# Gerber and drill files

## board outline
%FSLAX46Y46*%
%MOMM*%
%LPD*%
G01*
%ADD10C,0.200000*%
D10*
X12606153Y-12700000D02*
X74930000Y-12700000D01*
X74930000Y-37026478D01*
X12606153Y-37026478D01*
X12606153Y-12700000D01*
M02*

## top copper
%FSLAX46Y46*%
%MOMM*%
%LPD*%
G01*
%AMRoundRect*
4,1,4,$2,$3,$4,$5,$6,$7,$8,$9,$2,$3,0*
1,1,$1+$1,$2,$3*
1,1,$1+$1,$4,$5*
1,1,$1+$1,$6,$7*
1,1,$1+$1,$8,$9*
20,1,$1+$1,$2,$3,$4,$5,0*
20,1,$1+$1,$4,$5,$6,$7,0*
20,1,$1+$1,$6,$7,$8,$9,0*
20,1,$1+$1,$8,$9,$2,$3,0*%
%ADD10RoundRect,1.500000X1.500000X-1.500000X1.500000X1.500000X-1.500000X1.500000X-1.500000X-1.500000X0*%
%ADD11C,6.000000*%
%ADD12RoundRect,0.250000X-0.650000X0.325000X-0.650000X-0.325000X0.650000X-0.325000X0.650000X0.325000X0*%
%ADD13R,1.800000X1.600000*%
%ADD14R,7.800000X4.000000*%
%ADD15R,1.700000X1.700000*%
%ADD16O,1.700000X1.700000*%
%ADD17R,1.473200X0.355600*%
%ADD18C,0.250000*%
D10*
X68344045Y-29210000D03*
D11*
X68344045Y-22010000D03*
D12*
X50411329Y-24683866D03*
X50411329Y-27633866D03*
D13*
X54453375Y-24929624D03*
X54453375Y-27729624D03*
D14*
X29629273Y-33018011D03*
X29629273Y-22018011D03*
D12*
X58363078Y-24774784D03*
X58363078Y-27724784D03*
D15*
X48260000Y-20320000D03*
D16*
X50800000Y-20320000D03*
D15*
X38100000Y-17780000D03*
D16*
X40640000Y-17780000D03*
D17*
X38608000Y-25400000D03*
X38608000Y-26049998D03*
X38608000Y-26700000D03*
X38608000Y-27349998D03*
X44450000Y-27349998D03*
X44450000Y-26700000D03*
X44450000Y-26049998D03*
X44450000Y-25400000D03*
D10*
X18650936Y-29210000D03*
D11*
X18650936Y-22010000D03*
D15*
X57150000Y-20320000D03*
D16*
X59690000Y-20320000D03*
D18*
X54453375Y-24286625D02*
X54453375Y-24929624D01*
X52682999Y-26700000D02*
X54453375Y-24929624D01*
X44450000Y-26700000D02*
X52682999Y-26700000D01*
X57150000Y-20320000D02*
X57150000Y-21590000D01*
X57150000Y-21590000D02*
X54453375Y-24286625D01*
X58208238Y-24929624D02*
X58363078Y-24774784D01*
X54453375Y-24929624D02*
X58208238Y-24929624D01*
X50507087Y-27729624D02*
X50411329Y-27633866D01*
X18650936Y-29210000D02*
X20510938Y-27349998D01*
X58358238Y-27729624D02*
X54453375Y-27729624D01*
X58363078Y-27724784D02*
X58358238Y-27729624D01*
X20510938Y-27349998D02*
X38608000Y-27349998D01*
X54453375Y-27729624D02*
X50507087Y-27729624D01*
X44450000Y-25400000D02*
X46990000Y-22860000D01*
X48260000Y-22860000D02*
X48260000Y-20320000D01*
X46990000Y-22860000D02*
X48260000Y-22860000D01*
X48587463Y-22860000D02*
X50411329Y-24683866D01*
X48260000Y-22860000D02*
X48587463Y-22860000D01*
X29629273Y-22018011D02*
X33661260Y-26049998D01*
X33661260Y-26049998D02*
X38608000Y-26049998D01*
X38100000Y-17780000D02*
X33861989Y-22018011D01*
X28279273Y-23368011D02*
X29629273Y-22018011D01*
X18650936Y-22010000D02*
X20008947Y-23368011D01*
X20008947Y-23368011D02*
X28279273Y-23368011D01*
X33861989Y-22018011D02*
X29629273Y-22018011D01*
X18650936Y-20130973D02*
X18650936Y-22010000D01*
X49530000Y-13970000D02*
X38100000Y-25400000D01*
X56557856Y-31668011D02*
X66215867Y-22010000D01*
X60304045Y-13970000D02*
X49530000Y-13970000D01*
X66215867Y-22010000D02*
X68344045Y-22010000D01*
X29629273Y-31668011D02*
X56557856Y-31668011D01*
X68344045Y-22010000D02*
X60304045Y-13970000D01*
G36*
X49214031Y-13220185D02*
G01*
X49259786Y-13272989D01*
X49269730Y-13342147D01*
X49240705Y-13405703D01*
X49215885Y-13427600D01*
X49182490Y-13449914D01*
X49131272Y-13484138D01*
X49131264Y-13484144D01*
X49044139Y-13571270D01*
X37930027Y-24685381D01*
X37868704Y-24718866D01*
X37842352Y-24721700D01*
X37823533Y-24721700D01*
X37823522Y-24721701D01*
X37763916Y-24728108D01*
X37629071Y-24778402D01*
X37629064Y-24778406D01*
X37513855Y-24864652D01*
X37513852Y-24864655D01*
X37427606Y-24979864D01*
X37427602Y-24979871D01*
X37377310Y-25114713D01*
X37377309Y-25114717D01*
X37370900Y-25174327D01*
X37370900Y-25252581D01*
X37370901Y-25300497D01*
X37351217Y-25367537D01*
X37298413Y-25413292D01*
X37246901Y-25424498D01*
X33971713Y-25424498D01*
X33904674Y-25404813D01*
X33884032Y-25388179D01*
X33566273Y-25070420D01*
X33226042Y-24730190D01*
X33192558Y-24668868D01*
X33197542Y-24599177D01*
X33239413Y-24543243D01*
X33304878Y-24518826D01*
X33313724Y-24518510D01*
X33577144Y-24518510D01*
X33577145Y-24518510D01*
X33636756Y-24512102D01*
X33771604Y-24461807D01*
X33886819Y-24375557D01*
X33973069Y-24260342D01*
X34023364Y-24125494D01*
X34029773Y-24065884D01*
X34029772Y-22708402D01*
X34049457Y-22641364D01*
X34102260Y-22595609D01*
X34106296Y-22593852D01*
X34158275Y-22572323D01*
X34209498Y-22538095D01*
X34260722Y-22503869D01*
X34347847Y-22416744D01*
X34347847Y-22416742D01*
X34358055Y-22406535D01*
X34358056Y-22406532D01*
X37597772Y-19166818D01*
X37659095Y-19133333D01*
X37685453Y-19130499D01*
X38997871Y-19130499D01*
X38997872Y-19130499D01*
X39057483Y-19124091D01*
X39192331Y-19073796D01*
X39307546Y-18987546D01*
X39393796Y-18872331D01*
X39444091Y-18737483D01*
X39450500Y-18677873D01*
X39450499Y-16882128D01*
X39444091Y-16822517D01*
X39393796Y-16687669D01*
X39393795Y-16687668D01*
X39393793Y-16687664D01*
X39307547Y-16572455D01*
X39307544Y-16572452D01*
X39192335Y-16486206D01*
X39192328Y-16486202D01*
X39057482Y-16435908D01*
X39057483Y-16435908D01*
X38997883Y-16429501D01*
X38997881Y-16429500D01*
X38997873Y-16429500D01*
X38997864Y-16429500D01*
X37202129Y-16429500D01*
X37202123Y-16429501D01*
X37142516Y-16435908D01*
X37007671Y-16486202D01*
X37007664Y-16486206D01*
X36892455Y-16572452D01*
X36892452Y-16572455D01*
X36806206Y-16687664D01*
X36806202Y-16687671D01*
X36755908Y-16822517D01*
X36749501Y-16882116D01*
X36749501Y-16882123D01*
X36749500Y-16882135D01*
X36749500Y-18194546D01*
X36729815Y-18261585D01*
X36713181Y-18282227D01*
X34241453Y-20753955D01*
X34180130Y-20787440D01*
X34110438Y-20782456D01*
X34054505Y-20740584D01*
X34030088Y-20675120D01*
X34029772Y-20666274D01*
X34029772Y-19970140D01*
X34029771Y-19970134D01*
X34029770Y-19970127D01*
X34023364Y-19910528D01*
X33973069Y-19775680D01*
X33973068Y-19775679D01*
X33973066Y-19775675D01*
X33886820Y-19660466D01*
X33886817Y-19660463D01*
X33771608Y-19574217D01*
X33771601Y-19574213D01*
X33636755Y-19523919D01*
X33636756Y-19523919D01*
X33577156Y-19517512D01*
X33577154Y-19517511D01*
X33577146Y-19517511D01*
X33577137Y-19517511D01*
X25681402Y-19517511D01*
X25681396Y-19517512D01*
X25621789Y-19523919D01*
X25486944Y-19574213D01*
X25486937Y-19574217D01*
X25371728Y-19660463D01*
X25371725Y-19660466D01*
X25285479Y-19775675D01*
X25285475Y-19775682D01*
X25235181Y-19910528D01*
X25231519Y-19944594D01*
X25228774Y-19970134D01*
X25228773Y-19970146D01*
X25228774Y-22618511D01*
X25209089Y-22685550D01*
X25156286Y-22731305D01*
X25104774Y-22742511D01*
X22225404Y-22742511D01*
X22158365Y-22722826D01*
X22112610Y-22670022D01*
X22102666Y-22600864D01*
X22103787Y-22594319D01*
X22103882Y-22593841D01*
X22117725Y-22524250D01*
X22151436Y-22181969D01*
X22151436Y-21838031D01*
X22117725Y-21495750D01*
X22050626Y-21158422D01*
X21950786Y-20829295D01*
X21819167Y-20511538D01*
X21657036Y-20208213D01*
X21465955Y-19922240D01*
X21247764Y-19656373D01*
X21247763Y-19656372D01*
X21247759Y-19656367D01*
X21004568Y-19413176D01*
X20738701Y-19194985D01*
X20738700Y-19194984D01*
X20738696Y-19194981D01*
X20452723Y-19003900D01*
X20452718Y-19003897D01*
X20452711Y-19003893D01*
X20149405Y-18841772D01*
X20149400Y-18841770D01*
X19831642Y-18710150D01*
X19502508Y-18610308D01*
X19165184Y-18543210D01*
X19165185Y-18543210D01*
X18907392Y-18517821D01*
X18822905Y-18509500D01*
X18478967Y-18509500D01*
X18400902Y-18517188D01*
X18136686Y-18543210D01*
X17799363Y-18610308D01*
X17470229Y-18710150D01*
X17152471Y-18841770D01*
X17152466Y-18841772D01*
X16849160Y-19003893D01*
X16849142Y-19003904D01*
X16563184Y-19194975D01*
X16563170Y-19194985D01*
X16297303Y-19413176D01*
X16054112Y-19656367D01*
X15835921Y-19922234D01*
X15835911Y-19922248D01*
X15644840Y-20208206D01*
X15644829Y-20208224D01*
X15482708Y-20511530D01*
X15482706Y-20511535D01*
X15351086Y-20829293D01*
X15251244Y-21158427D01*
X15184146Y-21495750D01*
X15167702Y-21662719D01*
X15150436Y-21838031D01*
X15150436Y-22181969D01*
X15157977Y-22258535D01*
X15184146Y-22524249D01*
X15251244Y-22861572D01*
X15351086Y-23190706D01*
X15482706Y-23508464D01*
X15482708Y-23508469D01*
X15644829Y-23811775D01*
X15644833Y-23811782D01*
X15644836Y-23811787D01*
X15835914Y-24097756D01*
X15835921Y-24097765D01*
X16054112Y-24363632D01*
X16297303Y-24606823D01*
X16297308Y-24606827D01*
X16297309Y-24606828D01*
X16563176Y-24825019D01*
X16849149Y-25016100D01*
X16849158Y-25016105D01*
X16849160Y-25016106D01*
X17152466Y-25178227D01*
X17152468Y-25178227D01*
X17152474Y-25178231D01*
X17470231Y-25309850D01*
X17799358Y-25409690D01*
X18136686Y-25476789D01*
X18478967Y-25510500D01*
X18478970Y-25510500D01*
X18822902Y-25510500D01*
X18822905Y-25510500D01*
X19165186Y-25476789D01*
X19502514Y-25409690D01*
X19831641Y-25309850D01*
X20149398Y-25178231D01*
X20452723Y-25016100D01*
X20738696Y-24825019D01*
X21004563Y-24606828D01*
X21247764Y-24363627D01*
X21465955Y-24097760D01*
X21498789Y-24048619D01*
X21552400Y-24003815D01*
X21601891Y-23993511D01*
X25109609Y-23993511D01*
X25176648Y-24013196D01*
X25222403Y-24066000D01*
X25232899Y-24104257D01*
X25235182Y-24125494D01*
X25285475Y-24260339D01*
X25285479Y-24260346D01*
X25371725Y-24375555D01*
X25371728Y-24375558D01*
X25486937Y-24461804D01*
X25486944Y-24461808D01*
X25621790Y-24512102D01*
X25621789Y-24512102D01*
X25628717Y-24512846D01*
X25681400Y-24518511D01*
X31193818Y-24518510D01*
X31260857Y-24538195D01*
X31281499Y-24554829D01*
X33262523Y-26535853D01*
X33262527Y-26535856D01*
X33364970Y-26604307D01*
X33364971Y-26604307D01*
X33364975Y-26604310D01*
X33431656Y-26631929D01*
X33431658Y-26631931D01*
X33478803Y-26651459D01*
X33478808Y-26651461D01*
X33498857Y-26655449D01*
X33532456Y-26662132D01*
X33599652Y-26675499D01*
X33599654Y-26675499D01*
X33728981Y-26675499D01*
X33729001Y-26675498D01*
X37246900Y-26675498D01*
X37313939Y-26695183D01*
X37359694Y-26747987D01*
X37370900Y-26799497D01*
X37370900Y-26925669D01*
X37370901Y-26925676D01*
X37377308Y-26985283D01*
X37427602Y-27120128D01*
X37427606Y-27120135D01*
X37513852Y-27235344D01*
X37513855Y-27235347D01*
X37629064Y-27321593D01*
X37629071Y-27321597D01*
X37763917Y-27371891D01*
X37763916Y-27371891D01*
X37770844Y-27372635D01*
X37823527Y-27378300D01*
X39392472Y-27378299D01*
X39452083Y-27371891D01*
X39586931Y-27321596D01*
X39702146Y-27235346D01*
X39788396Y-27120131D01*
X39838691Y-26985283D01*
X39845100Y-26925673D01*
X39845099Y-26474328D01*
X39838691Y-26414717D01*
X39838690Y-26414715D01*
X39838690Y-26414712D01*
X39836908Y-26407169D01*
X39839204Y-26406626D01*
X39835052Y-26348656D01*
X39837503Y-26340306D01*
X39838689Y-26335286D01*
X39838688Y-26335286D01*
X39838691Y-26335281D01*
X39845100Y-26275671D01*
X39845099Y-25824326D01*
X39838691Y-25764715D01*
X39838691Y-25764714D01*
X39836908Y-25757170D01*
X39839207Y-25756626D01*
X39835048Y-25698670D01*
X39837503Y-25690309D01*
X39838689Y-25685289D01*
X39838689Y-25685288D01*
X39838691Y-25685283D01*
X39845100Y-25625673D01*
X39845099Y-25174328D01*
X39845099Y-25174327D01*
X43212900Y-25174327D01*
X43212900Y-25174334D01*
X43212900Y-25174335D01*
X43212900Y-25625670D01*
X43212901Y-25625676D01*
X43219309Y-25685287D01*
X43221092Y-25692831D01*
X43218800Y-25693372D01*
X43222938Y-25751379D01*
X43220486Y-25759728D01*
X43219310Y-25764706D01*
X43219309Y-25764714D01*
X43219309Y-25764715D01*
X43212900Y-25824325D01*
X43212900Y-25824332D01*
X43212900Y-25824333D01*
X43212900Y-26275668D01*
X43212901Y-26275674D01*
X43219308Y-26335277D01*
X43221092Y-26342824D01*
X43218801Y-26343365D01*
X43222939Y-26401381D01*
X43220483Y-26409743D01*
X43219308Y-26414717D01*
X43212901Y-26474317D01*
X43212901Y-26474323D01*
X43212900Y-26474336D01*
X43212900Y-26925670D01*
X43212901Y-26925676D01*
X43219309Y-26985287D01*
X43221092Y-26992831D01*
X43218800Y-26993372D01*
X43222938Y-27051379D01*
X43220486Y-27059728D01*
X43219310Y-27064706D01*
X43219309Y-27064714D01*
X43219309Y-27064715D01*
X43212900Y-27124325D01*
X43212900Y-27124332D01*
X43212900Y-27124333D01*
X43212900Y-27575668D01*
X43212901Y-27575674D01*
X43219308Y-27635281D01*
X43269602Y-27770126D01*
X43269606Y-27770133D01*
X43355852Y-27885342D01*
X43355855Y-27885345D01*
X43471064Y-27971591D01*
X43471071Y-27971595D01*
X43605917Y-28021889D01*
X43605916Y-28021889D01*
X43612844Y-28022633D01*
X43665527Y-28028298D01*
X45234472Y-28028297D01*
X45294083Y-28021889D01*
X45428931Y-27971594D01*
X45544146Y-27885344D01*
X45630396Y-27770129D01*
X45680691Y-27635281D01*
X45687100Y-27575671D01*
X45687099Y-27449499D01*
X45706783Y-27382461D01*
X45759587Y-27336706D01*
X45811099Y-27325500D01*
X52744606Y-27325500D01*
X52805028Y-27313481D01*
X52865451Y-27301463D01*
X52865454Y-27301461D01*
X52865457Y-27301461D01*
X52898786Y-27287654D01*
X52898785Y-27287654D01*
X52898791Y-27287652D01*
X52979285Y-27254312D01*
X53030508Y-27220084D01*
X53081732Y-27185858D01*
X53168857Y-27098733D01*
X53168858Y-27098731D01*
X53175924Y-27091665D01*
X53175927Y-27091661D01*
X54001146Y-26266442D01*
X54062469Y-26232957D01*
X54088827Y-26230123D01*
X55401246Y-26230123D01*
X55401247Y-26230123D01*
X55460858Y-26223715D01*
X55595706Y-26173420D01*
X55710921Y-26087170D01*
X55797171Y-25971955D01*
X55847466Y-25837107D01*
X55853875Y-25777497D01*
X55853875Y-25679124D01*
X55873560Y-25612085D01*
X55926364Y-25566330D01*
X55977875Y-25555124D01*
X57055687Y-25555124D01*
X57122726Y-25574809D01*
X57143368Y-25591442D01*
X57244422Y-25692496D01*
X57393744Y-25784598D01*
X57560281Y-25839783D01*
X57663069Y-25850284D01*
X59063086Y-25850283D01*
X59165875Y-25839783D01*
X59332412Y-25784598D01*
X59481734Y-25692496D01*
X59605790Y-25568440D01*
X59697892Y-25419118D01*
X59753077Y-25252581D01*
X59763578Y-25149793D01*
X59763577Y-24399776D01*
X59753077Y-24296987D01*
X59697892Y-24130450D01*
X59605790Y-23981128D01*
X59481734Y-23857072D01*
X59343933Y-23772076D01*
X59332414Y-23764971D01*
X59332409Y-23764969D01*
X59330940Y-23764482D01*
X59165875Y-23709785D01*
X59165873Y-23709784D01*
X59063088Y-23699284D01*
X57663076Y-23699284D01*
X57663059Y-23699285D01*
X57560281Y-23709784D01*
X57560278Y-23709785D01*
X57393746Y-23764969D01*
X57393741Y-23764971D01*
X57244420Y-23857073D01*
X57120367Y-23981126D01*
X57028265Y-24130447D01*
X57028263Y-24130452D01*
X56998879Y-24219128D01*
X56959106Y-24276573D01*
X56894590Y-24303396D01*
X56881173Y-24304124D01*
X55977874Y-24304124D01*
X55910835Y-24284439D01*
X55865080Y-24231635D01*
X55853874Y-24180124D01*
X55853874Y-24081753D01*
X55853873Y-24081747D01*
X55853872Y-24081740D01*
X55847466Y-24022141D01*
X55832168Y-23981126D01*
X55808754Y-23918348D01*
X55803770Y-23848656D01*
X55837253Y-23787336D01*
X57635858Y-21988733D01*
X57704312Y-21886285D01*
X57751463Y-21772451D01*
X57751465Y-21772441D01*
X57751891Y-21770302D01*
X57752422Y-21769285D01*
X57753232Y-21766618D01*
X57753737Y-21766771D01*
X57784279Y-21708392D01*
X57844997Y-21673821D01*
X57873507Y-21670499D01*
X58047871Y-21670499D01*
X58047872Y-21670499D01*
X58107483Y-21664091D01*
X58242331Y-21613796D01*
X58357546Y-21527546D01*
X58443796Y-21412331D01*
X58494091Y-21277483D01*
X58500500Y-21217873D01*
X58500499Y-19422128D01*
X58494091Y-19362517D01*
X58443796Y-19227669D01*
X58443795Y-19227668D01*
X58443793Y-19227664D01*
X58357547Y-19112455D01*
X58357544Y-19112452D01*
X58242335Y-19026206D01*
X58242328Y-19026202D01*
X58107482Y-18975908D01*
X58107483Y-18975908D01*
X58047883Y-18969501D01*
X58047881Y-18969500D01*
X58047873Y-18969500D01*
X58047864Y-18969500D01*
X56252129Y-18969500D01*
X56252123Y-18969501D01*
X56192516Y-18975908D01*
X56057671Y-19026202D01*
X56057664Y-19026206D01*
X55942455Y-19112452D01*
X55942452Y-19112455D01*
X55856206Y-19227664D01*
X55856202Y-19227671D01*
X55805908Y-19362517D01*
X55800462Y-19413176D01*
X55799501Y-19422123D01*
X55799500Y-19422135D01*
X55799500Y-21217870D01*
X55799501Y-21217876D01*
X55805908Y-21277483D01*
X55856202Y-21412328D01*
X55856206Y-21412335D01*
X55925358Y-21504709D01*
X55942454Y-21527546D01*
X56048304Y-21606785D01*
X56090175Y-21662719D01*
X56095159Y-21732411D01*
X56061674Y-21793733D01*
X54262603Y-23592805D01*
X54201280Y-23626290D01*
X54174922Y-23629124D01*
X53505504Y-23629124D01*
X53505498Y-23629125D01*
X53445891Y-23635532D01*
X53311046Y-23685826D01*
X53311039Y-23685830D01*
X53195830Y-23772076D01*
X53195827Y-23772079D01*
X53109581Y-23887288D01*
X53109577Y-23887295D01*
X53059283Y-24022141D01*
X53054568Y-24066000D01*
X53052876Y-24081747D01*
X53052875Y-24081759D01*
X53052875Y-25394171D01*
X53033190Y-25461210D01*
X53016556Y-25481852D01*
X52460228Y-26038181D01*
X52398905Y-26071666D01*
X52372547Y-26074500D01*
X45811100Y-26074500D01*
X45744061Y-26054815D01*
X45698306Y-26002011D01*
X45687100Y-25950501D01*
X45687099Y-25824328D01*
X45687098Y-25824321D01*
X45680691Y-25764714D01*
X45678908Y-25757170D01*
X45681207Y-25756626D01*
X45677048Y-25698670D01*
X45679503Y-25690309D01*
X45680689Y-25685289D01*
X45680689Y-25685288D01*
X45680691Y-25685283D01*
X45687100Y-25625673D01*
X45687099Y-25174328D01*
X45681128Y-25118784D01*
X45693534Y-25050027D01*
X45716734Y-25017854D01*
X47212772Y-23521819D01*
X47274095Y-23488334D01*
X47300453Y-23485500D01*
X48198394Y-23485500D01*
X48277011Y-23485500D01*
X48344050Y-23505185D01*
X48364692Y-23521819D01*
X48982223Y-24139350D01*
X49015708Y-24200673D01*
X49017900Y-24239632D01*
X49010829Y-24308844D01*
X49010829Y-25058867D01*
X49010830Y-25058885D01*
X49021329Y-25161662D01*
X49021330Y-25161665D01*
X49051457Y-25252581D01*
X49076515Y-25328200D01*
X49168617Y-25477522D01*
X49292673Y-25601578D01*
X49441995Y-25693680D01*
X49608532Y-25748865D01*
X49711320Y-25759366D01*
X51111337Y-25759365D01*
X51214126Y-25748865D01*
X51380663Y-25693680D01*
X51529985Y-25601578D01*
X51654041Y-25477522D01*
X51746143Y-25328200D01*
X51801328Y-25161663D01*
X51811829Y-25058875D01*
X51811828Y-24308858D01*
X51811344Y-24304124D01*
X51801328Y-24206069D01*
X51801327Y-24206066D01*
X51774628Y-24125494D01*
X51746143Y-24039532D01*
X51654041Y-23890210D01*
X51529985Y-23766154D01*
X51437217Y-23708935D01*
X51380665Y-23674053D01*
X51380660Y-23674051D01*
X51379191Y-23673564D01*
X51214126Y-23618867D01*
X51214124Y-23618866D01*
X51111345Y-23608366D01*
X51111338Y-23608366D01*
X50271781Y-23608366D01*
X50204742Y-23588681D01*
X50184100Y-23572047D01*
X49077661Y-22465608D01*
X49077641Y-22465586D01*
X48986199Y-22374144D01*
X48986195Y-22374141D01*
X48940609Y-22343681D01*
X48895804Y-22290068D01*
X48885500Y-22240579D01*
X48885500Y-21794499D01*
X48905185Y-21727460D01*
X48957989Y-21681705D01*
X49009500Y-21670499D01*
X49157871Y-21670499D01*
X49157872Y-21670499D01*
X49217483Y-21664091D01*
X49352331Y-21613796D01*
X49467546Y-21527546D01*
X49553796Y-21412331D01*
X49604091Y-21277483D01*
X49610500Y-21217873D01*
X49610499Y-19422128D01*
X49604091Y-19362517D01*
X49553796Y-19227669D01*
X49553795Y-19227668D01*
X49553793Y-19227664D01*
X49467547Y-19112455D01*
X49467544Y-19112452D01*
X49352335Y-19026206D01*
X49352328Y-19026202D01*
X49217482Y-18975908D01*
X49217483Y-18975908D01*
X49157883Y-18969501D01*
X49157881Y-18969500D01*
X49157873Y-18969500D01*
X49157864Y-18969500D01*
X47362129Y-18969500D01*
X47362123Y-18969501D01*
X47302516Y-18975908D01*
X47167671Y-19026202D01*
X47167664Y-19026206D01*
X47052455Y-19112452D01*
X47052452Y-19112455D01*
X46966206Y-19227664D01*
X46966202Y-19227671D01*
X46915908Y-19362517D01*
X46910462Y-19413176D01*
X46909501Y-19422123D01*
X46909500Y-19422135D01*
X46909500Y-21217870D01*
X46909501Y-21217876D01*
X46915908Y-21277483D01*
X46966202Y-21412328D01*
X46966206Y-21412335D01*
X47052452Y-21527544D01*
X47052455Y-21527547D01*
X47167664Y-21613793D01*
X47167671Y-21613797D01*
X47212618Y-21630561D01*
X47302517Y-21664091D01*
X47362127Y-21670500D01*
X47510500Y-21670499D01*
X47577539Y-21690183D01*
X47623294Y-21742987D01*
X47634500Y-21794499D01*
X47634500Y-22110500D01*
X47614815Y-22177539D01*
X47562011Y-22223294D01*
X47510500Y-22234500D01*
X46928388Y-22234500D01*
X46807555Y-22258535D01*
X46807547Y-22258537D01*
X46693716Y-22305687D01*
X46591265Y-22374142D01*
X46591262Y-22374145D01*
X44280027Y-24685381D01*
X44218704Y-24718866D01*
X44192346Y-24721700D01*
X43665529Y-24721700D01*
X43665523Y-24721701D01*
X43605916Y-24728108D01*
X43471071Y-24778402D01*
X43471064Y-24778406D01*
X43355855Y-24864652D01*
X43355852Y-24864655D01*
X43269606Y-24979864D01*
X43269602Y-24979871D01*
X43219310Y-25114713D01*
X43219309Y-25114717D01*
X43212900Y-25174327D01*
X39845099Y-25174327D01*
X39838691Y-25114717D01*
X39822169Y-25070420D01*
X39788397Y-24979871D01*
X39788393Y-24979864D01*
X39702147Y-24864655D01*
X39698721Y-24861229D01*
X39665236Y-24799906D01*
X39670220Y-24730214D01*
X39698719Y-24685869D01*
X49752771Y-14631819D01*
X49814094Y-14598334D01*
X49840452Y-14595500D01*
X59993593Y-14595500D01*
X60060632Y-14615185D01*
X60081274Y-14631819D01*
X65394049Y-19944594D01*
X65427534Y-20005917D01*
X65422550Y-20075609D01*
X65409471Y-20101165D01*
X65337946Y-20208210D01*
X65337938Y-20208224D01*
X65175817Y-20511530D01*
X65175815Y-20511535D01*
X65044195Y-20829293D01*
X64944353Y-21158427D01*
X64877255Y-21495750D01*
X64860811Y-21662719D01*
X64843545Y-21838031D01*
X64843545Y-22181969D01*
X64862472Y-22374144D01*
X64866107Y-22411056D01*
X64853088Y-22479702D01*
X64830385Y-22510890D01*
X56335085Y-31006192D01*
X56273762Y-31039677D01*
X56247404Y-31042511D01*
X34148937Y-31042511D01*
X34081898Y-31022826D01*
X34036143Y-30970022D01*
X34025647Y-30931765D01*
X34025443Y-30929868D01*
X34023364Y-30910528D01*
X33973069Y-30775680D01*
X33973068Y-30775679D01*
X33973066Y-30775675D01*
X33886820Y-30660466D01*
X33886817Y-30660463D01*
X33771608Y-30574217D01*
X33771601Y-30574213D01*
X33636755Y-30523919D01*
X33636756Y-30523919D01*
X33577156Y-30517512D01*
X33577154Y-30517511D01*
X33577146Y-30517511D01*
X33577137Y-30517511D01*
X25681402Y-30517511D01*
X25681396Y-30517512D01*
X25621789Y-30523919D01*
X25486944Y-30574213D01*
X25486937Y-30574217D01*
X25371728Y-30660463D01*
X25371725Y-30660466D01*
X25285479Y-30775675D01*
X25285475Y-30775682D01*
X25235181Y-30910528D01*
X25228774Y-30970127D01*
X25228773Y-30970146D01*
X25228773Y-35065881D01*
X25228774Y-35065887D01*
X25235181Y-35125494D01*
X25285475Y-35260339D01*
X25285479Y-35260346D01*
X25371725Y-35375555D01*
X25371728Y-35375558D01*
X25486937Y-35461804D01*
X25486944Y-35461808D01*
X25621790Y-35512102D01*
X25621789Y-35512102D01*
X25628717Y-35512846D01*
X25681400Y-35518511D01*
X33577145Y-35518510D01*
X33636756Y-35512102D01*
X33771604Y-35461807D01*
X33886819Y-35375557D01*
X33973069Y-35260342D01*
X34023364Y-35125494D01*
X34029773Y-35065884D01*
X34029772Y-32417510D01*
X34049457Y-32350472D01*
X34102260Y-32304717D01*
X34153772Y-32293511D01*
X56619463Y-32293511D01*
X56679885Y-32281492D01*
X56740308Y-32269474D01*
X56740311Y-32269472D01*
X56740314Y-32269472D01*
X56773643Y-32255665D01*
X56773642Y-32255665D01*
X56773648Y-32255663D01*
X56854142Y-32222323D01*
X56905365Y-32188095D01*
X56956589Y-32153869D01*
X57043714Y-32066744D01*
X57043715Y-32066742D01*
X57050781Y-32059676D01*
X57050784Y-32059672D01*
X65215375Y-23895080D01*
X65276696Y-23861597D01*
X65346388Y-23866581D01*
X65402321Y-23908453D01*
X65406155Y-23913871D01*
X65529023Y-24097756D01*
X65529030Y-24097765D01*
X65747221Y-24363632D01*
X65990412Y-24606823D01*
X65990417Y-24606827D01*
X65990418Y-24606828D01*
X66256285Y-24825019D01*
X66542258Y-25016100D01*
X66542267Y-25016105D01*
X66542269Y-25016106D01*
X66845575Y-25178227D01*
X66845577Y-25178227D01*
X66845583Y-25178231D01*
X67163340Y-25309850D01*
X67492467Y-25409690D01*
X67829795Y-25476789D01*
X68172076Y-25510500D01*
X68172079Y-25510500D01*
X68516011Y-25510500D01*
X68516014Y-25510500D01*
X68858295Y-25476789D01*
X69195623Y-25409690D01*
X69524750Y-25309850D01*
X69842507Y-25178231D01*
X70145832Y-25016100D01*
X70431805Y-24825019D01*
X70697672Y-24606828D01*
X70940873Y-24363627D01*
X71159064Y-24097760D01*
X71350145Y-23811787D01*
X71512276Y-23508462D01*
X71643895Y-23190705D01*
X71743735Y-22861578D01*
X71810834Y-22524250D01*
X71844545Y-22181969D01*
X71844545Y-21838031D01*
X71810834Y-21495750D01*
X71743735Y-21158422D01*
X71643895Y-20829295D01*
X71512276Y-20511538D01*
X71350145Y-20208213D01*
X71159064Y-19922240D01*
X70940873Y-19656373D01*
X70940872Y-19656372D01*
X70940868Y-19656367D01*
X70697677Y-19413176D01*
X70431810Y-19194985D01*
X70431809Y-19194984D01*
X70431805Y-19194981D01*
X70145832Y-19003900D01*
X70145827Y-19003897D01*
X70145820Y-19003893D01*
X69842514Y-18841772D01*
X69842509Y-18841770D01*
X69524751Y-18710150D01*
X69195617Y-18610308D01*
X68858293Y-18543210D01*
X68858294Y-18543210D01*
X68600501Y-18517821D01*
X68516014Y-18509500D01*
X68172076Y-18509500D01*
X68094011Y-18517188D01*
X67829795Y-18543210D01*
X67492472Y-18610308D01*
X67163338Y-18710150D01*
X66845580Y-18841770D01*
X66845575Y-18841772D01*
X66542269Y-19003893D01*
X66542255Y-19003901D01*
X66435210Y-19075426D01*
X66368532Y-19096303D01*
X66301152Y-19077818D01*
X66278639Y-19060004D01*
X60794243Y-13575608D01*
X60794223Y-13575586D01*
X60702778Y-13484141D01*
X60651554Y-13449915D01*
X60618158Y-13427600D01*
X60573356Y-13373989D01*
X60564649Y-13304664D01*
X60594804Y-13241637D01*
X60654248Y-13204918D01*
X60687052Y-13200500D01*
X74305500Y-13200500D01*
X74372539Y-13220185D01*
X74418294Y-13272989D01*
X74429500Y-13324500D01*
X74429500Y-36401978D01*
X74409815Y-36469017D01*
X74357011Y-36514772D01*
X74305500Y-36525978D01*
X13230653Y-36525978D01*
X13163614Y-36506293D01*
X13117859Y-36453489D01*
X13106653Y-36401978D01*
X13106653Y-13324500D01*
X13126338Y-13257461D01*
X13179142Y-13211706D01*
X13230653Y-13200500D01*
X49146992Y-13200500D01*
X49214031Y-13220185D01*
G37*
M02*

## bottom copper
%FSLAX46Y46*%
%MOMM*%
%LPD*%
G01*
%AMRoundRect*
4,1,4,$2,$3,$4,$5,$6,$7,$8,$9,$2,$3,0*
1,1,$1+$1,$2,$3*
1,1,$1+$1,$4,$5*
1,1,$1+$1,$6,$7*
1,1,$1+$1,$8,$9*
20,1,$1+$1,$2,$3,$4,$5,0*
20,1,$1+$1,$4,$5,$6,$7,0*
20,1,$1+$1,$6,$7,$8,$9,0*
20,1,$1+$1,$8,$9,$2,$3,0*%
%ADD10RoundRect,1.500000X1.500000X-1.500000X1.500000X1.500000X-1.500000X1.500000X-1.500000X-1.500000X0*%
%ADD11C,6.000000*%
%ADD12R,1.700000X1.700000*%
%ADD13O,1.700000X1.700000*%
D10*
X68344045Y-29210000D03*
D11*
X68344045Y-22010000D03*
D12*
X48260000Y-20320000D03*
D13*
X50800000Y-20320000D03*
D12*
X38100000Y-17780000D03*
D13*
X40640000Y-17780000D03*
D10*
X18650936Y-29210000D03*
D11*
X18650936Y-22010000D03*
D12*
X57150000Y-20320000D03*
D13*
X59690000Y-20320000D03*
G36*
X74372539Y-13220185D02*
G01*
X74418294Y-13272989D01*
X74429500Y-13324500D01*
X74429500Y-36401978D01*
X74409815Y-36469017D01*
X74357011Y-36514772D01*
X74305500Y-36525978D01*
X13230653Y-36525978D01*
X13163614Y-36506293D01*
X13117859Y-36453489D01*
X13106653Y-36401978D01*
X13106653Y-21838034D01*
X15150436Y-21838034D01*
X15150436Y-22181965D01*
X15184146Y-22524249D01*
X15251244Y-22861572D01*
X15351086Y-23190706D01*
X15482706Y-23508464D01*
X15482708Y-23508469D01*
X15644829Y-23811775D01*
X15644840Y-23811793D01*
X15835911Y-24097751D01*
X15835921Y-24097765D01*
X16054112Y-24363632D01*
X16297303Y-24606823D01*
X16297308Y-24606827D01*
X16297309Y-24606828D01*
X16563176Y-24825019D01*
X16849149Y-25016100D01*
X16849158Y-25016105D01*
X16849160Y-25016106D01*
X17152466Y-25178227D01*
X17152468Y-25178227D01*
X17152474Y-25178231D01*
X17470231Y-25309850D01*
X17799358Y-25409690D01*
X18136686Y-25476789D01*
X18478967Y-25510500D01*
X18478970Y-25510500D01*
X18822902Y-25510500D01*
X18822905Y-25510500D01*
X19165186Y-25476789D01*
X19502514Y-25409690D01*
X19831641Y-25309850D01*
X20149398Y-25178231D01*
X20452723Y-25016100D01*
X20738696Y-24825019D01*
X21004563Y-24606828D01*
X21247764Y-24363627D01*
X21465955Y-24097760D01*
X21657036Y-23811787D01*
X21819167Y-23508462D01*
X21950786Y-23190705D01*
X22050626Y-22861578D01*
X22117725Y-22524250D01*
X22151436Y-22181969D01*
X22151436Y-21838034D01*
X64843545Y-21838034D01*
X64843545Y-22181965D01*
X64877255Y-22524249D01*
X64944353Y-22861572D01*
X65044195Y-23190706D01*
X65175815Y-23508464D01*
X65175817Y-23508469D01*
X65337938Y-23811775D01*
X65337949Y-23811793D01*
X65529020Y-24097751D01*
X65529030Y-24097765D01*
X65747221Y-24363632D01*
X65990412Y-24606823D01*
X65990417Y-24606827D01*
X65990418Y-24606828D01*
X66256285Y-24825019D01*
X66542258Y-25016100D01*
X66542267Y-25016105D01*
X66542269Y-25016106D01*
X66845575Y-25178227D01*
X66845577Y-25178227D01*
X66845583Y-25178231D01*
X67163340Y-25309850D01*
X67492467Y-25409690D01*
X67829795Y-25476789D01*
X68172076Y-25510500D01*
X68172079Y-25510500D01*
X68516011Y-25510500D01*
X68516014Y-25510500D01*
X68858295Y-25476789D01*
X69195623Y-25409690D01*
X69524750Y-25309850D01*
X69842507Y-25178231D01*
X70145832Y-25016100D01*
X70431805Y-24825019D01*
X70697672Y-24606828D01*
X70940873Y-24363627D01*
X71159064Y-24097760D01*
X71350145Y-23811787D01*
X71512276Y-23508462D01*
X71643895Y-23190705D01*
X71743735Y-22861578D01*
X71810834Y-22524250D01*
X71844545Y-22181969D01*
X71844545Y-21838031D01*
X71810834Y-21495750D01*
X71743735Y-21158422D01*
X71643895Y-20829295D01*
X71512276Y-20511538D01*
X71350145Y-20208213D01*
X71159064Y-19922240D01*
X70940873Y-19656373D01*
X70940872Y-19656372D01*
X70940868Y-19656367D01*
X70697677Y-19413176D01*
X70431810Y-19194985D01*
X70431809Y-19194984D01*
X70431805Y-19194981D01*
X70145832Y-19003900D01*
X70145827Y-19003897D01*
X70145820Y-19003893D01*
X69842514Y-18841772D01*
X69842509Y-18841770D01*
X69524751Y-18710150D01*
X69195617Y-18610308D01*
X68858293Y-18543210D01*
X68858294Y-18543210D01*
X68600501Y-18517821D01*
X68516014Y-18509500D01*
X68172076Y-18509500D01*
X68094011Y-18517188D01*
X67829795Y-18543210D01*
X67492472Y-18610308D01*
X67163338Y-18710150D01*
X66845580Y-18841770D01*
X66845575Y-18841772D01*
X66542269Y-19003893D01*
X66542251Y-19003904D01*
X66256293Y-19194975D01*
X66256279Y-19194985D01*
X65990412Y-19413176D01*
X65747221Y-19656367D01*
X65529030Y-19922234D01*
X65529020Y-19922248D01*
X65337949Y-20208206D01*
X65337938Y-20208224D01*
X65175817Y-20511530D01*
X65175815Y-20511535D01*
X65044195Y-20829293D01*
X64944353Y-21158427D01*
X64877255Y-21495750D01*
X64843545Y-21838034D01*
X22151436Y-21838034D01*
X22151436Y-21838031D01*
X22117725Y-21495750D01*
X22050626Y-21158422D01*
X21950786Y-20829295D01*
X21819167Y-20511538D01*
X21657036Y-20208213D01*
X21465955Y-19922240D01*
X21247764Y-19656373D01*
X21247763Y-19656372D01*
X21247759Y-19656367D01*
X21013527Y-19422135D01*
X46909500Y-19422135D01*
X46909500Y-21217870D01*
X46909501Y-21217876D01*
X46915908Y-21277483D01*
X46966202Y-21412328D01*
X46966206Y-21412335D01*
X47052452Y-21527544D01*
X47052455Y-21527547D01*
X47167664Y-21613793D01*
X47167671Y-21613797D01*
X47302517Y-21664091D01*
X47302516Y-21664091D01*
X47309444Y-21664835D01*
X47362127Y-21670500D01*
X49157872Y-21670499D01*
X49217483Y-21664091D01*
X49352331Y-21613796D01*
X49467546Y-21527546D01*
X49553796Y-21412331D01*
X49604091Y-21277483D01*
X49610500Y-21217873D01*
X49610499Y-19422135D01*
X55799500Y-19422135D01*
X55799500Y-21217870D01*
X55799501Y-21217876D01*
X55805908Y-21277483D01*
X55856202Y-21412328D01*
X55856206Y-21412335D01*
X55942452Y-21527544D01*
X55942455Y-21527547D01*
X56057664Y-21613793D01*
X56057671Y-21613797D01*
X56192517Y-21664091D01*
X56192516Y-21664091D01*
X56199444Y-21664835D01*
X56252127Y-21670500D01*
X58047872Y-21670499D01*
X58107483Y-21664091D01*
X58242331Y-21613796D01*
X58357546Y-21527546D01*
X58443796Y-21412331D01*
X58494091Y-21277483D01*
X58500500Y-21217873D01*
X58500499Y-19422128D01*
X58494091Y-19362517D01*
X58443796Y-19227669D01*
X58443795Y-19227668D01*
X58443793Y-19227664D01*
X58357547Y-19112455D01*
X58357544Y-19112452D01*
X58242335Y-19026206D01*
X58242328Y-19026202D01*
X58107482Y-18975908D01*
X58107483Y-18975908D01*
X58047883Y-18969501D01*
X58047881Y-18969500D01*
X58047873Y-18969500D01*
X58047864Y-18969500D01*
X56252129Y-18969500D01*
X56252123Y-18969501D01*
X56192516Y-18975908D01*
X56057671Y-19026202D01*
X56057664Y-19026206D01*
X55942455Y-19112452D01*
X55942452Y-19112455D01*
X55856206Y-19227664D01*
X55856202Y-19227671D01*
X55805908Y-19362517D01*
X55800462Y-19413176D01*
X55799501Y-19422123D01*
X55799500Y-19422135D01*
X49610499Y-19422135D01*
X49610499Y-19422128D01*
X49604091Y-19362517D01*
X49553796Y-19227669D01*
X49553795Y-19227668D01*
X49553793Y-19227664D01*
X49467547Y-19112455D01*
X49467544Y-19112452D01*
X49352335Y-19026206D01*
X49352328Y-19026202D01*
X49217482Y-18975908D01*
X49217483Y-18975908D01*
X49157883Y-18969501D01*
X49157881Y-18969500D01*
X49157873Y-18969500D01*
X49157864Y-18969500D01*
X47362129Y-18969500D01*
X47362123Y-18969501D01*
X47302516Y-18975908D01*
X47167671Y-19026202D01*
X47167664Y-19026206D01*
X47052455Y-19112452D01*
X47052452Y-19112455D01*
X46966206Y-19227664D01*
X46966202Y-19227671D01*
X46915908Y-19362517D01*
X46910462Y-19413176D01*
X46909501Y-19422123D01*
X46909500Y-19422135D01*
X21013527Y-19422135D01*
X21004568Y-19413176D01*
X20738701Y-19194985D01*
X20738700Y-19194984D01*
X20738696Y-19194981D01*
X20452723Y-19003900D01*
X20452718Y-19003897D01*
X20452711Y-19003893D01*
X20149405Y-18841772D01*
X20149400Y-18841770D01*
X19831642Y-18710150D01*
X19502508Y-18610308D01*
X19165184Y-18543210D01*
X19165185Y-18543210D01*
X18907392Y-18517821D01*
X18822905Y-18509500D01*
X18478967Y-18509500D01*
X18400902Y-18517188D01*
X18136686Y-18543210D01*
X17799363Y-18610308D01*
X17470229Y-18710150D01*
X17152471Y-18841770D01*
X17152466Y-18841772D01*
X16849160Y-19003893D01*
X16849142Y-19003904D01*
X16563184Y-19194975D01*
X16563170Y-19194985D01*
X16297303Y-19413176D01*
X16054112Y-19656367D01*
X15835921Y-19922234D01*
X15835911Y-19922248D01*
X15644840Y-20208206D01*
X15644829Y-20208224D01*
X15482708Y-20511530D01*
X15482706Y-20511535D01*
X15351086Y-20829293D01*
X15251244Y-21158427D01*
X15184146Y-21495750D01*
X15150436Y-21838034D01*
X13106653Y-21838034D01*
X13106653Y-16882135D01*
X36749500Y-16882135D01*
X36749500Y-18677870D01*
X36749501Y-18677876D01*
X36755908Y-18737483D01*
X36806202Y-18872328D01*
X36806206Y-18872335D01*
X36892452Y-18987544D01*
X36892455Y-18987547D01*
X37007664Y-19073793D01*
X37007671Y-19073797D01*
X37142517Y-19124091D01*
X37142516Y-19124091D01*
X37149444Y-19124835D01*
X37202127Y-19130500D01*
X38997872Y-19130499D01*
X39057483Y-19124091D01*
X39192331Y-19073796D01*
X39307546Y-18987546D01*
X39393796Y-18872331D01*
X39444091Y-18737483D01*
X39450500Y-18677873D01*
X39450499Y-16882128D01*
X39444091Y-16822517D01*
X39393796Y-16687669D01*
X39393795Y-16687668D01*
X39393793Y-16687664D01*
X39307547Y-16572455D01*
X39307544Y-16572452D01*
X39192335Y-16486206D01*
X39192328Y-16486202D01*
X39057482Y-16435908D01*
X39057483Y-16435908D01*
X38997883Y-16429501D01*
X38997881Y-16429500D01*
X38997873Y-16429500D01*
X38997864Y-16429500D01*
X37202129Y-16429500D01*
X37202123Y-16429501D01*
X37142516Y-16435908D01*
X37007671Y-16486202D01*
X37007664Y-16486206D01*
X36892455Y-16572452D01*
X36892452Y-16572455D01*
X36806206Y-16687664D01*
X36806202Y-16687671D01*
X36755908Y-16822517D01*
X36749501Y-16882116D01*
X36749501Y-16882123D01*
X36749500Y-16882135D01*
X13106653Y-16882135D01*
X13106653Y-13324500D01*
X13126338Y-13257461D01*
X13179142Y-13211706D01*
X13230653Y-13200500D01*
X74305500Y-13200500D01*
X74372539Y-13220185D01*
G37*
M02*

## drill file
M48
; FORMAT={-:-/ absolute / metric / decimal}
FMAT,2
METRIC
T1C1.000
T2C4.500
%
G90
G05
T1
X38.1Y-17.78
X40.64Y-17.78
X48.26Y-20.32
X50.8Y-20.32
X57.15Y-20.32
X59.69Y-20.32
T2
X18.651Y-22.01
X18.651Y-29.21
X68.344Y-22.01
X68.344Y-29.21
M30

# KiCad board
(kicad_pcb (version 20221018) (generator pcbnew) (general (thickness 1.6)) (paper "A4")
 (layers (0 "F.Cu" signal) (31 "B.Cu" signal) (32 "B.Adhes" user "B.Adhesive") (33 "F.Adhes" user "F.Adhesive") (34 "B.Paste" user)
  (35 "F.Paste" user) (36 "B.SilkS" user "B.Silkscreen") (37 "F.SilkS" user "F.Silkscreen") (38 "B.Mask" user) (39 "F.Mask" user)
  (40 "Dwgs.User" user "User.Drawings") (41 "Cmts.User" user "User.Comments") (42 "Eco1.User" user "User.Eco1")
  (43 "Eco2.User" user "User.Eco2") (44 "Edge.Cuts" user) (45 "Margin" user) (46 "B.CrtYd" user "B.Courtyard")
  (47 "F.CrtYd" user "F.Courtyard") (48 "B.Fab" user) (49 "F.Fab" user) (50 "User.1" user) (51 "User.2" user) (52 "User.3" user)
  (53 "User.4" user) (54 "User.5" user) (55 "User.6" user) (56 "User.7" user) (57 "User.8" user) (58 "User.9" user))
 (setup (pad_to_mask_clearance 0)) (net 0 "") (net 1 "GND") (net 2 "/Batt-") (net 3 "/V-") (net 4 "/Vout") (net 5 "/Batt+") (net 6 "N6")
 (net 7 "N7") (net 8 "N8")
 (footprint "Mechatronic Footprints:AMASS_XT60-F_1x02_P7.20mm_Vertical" (layer "F.Cu") (at 68.344045 29.21 90)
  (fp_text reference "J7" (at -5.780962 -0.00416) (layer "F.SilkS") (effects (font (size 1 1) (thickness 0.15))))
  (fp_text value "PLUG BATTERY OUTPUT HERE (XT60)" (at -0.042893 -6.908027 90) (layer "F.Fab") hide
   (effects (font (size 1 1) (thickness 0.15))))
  (pad "1" thru_hole roundrect (at 0 0 90) (size 6 6) (drill 4.5) (layers "*.Cu" "*.Mask") (roundrect_rratio 0.25) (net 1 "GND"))
  (pad "2" thru_hole circle (at 7.2 0 90) (size 6 6) (drill 4.5) (layers "*.Cu" "*.Mask") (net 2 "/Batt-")))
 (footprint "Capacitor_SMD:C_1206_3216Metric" (layer "F.Cu") (at 50.411329 26.158866 -90)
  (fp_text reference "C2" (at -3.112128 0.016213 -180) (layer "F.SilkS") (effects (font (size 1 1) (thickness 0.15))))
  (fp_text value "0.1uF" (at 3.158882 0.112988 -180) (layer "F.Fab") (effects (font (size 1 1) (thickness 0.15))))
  (pad "1" smd roundrect (at -1.475 0 270) (size 1.15 1.8) (layers "F.Cu" "F.Paste" "F.Mask") (roundrect_rratio 0.2173913043) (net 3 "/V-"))
  (pad "2" smd roundrect (at 1.475 0 270) (size 1.15 1.8) (layers "F.Cu" "F.Paste" "F.Mask") (roundrect_rratio 0.2173913043) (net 1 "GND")))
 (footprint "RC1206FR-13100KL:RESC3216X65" (layer "F.Cu") (at 54.453375 26.329624 -90)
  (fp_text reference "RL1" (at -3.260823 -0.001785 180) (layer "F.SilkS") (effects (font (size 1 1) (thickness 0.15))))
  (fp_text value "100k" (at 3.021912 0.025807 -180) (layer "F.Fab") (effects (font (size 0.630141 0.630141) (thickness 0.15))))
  (pad "1" smd rect (at -1.4 0 270) (size 1.6 1.8) (layers "F.Cu" "F.Paste" "F.Mask") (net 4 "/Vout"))
  (pad "2" smd rect (at 1.4 0 270) (size 1.6 1.8) (layers "F.Cu" "F.Paste" "F.Mask") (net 1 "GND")))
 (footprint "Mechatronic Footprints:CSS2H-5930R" (layer "F.Cu") (at 29.629273 27.518011 90)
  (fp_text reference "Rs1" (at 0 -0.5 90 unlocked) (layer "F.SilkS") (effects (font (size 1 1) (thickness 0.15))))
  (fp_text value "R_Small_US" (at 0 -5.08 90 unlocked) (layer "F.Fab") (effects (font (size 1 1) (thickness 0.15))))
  (pad "1" smd rect (at -5.5 0 180) (size 7.8 4) (layers "F.Cu" "F.Paste" "F.Mask") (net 2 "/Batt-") (thermal_bridge_angle 45))
  (pad "2" smd rect (at 5.5 0 180) (size 7.8 4) (layers "F.Cu" "F.Paste" "F.Mask") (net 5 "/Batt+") (thermal_bridge_angle 45)))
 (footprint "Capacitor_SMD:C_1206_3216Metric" (layer "F.Cu") (at 58.363078 26.249784 -90)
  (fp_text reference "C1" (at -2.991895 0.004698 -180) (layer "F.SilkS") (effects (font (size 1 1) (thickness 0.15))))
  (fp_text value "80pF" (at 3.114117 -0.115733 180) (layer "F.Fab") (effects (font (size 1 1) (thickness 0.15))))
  (pad "1" smd roundrect (at -1.475 0 270) (size 1.15 1.8) (layers "F.Cu" "F.Paste" "F.Mask") (roundrect_rratio 0.2173913043)
   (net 4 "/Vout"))
  (pad "2" smd roundrect (at 1.475 0 270) (size 1.15 1.8) (layers "F.Cu" "F.Paste" "F.Mask") (roundrect_rratio 0.2173913043) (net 1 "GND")))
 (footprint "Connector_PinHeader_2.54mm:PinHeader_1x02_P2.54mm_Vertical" (layer "F.Cu") (at 48.26 20.32 90)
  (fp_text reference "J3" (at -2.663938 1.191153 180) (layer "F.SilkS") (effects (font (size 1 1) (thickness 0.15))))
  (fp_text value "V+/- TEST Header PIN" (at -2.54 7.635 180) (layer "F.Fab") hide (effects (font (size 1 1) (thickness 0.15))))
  (pad "1" thru_hole rect (at 0 0 90) (size 1.7 1.7) (drill 1) (layers "*.Cu" "*.Mask") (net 3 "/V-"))
  (pad "2" thru_hole oval (at 0 2.54 90) (size 1.7 1.7) (drill 1) (layers "*.Cu" "*.Mask") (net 1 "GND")))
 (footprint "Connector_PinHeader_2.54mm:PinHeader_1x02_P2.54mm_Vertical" (layer "F.Cu") (at 38.1 17.78 90)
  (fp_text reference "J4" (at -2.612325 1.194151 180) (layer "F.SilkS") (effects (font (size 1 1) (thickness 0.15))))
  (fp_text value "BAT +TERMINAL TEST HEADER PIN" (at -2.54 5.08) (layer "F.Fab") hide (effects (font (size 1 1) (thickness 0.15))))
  (pad "1" thru_hole rect (at 0 0 90) (size 1.7 1.7) (drill 1) (layers "*.Cu" "*.Mask") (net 5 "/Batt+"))
  (pad "2" thru_hole oval (at 0 2.54 90) (size 1.7 1.7) (drill 1) (layers "*.Cu" "*.Mask") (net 1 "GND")))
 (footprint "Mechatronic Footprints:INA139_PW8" (layer "F.Cu") (at 41.529 26.374999)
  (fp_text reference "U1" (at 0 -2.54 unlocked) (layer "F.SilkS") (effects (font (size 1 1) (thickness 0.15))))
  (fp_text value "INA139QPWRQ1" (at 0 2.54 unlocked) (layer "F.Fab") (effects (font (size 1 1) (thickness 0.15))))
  (pad "1" smd rect (at -2.921 -0.974999) (size 1.4732 0.3556) (layers "F.Cu" "F.Paste" "F.Mask") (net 2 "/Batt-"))
  (pad "2" smd rect (at -2.921 -0.325001) (size 1.4732 0.3556) (layers "F.Cu" "F.Paste" "F.Mask") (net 5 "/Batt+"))
  (pad "3" smd rect (at -2.921 0.325001) (size 1.4732 0.3556) (layers "F.Cu" "F.Paste" "F.Mask") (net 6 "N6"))
  (pad "4" smd rect (at -2.921 0.974999) (size 1.4732 0.3556) (layers "F.Cu" "F.Paste" "F.Mask") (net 1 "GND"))
  (pad "5" smd rect (at 2.921 0.974999) (size 1.4732 0.3556) (layers "F.Cu" "F.Paste" "F.Mask") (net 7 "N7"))
  (pad "6" smd rect (at 2.921 0.325001) (size 1.4732 0.3556) (layers "F.Cu" "F.Paste" "F.Mask") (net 4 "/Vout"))
  (pad "7" smd rect (at 2.921 -0.325001) (size 1.4732 0.3556) (layers "F.Cu" "F.Paste" "F.Mask") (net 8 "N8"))
  (pad "8" smd rect (at 2.921 -0.974999) (size 1.4732 0.3556) (layers "F.Cu" "F.Paste" "F.Mask") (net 3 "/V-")))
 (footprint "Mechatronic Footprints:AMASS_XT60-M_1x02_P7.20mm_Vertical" (layer "F.Cu") (at 18.650936 29.21 90)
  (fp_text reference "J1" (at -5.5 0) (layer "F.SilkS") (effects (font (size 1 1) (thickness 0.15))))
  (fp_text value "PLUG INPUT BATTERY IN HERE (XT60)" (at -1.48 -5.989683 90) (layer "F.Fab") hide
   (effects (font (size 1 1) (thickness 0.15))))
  (pad "1" thru_hole roundrect (at 0 0 90) (size 6 6) (drill 4.5) (layers "*.Cu" "*.Mask") (roundrect_rratio 0.25) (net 1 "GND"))
  (pad "2" thru_hole circle (at 7.2 0 90) (size 6 6) (drill 4.5) (layers "*.Cu" "*.Mask") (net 5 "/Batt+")))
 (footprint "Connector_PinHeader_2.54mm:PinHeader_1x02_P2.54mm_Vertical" (layer "F.Cu") (at 57.15 20.32 90)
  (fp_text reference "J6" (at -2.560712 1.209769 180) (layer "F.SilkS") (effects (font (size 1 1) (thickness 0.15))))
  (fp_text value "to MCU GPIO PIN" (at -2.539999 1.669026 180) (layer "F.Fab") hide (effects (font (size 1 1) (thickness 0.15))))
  (pad "1" thru_hole rect (at 0 0 90) (size 1.7 1.7) (drill 1) (layers "*.Cu" "*.Mask") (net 4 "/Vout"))
  (pad "2" thru_hole oval (at 0 2.54 90) (size 1.7 1.7) (drill 1) (layers "*.Cu" "*.Mask") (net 1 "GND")))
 (gr_rect (start 12.606153 12.7) (end 74.93 37.026478) (stroke (width 0.2) (type default)) (fill none) (layer "Edge.Cuts"))
 (segment (start 54.453375 24.286625) (end 54.453375 24.929624) (width 0.25) (layer "F.Cu") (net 4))
 (segment (start 52.682999 26.7) (end 54.453375 24.929624) (width 0.25) (layer "F.Cu") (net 4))
 (segment (start 44.45 26.7) (end 52.682999 26.7) (width 0.25) (layer "F.Cu") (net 4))
 (segment (start 57.15 20.32) (end 57.15 21.59) (width 0.25) (layer "F.Cu") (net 4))
 (segment (start 57.15 21.59) (end 54.453375 24.286625) (width 0.25) (layer "F.Cu") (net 4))
 (segment (start 58.208238 24.929624) (end 58.363078 24.774784) (width 0.25) (layer "F.Cu") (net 4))
 (segment (start 54.453375 24.929624) (end 58.208238 24.929624) (width 0.25) (layer "F.Cu") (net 4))
 (segment (start 50.507087 27.729624) (end 50.411329 27.633866) (width 0.25) (layer "F.Cu") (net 1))
 (segment (start 18.650936 29.21) (end 20.510938 27.349998) (width 0.25) (layer "F.Cu") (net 1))
 (segment (start 58.358238 27.729624) (end 54.453375 27.729624) (width 0.25) (layer "F.Cu") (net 1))
 (segment (start 58.363078 27.724784) (end 58.358238 27.729624) (width 0.25) (layer "F.Cu") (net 1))
 (segment (start 20.510938 27.349998) (end 38.608 27.349998) (width 0.25) (layer "F.Cu") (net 1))
 (segment (start 54.453375 27.729624) (end 50.507087 27.729624) (width 0.25) (layer "F.Cu") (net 1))
 (segment (start 44.45 25.4) (end 46.99 22.86) (width 0.25) (layer "F.Cu") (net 3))
 (segment (start 48.26 22.86) (end 48.26 20.32) (width 0.25) (layer "F.Cu") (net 3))
 (segment (start 46.99 22.86) (end 48.26 22.86) (width 0.25) (layer "F.Cu") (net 3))
 (segment (start 48.587463 22.86) (end 50.411329 24.683866) (width 0.25) (layer "F.Cu") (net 3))
 (segment (start 48.26 22.86) (end 48.587463 22.86) (width 0.25) (layer "F.Cu") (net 3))
 (segment (start 29.629273 22.018011) (end 33.66126 26.049998) (width 0.25) (layer "F.Cu") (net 5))
 (segment (start 33.66126 26.049998) (end 38.608 26.049998) (width 0.25) (layer "F.Cu") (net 5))
 (segment (start 38.1 17.78) (end 33.861989 22.018011) (width 0.25) (layer "F.Cu") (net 5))
 (segment (start 28.279273 23.368011) (end 29.629273 22.018011) (width 0.25) (layer "F.Cu") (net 5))
 (segment (start 18.650936 22.01) (end 20.008947 23.368011) (width 0.25) (layer "F.Cu") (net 5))
 (segment (start 20.008947 23.368011) (end 28.279273 23.368011) (width 0.25) (layer "F.Cu") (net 5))
 (segment (start 33.861989 22.018011) (end 29.629273 22.018011) (width 0.25) (layer "F.Cu") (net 5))
 (segment (start 18.650936 20.130973) (end 18.650936 22.01) (width 0.25) (layer "F.Cu") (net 5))
 (segment (start 49.53 13.97) (end 38.1 25.4) (width 0.25) (layer "F.Cu") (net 2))
 (segment (start 56.557856 31.668011) (end 66.215867 22.01) (width 0.25) (layer "F.Cu") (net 2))
 (segment (start 60.304045 13.97) (end 49.53 13.97) (width 0.25) (layer "F.Cu") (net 2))
 (segment (start 66.215867 22.01) (end 68.344045 22.01) (width 0.25) (layer "F.Cu") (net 2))
 (segment (start 29.629273 31.668011) (end 56.557856 31.668011) (width 0.25) (layer "F.Cu") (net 2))
 (segment (start 68.344045 22.01) (end 60.304045 13.97) (width 0.25) (layer "F.Cu") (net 2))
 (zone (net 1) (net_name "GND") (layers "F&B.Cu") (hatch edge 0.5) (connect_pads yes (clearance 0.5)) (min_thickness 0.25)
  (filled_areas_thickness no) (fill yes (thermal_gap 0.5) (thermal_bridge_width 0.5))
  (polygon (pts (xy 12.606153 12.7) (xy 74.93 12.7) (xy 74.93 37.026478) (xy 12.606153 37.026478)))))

